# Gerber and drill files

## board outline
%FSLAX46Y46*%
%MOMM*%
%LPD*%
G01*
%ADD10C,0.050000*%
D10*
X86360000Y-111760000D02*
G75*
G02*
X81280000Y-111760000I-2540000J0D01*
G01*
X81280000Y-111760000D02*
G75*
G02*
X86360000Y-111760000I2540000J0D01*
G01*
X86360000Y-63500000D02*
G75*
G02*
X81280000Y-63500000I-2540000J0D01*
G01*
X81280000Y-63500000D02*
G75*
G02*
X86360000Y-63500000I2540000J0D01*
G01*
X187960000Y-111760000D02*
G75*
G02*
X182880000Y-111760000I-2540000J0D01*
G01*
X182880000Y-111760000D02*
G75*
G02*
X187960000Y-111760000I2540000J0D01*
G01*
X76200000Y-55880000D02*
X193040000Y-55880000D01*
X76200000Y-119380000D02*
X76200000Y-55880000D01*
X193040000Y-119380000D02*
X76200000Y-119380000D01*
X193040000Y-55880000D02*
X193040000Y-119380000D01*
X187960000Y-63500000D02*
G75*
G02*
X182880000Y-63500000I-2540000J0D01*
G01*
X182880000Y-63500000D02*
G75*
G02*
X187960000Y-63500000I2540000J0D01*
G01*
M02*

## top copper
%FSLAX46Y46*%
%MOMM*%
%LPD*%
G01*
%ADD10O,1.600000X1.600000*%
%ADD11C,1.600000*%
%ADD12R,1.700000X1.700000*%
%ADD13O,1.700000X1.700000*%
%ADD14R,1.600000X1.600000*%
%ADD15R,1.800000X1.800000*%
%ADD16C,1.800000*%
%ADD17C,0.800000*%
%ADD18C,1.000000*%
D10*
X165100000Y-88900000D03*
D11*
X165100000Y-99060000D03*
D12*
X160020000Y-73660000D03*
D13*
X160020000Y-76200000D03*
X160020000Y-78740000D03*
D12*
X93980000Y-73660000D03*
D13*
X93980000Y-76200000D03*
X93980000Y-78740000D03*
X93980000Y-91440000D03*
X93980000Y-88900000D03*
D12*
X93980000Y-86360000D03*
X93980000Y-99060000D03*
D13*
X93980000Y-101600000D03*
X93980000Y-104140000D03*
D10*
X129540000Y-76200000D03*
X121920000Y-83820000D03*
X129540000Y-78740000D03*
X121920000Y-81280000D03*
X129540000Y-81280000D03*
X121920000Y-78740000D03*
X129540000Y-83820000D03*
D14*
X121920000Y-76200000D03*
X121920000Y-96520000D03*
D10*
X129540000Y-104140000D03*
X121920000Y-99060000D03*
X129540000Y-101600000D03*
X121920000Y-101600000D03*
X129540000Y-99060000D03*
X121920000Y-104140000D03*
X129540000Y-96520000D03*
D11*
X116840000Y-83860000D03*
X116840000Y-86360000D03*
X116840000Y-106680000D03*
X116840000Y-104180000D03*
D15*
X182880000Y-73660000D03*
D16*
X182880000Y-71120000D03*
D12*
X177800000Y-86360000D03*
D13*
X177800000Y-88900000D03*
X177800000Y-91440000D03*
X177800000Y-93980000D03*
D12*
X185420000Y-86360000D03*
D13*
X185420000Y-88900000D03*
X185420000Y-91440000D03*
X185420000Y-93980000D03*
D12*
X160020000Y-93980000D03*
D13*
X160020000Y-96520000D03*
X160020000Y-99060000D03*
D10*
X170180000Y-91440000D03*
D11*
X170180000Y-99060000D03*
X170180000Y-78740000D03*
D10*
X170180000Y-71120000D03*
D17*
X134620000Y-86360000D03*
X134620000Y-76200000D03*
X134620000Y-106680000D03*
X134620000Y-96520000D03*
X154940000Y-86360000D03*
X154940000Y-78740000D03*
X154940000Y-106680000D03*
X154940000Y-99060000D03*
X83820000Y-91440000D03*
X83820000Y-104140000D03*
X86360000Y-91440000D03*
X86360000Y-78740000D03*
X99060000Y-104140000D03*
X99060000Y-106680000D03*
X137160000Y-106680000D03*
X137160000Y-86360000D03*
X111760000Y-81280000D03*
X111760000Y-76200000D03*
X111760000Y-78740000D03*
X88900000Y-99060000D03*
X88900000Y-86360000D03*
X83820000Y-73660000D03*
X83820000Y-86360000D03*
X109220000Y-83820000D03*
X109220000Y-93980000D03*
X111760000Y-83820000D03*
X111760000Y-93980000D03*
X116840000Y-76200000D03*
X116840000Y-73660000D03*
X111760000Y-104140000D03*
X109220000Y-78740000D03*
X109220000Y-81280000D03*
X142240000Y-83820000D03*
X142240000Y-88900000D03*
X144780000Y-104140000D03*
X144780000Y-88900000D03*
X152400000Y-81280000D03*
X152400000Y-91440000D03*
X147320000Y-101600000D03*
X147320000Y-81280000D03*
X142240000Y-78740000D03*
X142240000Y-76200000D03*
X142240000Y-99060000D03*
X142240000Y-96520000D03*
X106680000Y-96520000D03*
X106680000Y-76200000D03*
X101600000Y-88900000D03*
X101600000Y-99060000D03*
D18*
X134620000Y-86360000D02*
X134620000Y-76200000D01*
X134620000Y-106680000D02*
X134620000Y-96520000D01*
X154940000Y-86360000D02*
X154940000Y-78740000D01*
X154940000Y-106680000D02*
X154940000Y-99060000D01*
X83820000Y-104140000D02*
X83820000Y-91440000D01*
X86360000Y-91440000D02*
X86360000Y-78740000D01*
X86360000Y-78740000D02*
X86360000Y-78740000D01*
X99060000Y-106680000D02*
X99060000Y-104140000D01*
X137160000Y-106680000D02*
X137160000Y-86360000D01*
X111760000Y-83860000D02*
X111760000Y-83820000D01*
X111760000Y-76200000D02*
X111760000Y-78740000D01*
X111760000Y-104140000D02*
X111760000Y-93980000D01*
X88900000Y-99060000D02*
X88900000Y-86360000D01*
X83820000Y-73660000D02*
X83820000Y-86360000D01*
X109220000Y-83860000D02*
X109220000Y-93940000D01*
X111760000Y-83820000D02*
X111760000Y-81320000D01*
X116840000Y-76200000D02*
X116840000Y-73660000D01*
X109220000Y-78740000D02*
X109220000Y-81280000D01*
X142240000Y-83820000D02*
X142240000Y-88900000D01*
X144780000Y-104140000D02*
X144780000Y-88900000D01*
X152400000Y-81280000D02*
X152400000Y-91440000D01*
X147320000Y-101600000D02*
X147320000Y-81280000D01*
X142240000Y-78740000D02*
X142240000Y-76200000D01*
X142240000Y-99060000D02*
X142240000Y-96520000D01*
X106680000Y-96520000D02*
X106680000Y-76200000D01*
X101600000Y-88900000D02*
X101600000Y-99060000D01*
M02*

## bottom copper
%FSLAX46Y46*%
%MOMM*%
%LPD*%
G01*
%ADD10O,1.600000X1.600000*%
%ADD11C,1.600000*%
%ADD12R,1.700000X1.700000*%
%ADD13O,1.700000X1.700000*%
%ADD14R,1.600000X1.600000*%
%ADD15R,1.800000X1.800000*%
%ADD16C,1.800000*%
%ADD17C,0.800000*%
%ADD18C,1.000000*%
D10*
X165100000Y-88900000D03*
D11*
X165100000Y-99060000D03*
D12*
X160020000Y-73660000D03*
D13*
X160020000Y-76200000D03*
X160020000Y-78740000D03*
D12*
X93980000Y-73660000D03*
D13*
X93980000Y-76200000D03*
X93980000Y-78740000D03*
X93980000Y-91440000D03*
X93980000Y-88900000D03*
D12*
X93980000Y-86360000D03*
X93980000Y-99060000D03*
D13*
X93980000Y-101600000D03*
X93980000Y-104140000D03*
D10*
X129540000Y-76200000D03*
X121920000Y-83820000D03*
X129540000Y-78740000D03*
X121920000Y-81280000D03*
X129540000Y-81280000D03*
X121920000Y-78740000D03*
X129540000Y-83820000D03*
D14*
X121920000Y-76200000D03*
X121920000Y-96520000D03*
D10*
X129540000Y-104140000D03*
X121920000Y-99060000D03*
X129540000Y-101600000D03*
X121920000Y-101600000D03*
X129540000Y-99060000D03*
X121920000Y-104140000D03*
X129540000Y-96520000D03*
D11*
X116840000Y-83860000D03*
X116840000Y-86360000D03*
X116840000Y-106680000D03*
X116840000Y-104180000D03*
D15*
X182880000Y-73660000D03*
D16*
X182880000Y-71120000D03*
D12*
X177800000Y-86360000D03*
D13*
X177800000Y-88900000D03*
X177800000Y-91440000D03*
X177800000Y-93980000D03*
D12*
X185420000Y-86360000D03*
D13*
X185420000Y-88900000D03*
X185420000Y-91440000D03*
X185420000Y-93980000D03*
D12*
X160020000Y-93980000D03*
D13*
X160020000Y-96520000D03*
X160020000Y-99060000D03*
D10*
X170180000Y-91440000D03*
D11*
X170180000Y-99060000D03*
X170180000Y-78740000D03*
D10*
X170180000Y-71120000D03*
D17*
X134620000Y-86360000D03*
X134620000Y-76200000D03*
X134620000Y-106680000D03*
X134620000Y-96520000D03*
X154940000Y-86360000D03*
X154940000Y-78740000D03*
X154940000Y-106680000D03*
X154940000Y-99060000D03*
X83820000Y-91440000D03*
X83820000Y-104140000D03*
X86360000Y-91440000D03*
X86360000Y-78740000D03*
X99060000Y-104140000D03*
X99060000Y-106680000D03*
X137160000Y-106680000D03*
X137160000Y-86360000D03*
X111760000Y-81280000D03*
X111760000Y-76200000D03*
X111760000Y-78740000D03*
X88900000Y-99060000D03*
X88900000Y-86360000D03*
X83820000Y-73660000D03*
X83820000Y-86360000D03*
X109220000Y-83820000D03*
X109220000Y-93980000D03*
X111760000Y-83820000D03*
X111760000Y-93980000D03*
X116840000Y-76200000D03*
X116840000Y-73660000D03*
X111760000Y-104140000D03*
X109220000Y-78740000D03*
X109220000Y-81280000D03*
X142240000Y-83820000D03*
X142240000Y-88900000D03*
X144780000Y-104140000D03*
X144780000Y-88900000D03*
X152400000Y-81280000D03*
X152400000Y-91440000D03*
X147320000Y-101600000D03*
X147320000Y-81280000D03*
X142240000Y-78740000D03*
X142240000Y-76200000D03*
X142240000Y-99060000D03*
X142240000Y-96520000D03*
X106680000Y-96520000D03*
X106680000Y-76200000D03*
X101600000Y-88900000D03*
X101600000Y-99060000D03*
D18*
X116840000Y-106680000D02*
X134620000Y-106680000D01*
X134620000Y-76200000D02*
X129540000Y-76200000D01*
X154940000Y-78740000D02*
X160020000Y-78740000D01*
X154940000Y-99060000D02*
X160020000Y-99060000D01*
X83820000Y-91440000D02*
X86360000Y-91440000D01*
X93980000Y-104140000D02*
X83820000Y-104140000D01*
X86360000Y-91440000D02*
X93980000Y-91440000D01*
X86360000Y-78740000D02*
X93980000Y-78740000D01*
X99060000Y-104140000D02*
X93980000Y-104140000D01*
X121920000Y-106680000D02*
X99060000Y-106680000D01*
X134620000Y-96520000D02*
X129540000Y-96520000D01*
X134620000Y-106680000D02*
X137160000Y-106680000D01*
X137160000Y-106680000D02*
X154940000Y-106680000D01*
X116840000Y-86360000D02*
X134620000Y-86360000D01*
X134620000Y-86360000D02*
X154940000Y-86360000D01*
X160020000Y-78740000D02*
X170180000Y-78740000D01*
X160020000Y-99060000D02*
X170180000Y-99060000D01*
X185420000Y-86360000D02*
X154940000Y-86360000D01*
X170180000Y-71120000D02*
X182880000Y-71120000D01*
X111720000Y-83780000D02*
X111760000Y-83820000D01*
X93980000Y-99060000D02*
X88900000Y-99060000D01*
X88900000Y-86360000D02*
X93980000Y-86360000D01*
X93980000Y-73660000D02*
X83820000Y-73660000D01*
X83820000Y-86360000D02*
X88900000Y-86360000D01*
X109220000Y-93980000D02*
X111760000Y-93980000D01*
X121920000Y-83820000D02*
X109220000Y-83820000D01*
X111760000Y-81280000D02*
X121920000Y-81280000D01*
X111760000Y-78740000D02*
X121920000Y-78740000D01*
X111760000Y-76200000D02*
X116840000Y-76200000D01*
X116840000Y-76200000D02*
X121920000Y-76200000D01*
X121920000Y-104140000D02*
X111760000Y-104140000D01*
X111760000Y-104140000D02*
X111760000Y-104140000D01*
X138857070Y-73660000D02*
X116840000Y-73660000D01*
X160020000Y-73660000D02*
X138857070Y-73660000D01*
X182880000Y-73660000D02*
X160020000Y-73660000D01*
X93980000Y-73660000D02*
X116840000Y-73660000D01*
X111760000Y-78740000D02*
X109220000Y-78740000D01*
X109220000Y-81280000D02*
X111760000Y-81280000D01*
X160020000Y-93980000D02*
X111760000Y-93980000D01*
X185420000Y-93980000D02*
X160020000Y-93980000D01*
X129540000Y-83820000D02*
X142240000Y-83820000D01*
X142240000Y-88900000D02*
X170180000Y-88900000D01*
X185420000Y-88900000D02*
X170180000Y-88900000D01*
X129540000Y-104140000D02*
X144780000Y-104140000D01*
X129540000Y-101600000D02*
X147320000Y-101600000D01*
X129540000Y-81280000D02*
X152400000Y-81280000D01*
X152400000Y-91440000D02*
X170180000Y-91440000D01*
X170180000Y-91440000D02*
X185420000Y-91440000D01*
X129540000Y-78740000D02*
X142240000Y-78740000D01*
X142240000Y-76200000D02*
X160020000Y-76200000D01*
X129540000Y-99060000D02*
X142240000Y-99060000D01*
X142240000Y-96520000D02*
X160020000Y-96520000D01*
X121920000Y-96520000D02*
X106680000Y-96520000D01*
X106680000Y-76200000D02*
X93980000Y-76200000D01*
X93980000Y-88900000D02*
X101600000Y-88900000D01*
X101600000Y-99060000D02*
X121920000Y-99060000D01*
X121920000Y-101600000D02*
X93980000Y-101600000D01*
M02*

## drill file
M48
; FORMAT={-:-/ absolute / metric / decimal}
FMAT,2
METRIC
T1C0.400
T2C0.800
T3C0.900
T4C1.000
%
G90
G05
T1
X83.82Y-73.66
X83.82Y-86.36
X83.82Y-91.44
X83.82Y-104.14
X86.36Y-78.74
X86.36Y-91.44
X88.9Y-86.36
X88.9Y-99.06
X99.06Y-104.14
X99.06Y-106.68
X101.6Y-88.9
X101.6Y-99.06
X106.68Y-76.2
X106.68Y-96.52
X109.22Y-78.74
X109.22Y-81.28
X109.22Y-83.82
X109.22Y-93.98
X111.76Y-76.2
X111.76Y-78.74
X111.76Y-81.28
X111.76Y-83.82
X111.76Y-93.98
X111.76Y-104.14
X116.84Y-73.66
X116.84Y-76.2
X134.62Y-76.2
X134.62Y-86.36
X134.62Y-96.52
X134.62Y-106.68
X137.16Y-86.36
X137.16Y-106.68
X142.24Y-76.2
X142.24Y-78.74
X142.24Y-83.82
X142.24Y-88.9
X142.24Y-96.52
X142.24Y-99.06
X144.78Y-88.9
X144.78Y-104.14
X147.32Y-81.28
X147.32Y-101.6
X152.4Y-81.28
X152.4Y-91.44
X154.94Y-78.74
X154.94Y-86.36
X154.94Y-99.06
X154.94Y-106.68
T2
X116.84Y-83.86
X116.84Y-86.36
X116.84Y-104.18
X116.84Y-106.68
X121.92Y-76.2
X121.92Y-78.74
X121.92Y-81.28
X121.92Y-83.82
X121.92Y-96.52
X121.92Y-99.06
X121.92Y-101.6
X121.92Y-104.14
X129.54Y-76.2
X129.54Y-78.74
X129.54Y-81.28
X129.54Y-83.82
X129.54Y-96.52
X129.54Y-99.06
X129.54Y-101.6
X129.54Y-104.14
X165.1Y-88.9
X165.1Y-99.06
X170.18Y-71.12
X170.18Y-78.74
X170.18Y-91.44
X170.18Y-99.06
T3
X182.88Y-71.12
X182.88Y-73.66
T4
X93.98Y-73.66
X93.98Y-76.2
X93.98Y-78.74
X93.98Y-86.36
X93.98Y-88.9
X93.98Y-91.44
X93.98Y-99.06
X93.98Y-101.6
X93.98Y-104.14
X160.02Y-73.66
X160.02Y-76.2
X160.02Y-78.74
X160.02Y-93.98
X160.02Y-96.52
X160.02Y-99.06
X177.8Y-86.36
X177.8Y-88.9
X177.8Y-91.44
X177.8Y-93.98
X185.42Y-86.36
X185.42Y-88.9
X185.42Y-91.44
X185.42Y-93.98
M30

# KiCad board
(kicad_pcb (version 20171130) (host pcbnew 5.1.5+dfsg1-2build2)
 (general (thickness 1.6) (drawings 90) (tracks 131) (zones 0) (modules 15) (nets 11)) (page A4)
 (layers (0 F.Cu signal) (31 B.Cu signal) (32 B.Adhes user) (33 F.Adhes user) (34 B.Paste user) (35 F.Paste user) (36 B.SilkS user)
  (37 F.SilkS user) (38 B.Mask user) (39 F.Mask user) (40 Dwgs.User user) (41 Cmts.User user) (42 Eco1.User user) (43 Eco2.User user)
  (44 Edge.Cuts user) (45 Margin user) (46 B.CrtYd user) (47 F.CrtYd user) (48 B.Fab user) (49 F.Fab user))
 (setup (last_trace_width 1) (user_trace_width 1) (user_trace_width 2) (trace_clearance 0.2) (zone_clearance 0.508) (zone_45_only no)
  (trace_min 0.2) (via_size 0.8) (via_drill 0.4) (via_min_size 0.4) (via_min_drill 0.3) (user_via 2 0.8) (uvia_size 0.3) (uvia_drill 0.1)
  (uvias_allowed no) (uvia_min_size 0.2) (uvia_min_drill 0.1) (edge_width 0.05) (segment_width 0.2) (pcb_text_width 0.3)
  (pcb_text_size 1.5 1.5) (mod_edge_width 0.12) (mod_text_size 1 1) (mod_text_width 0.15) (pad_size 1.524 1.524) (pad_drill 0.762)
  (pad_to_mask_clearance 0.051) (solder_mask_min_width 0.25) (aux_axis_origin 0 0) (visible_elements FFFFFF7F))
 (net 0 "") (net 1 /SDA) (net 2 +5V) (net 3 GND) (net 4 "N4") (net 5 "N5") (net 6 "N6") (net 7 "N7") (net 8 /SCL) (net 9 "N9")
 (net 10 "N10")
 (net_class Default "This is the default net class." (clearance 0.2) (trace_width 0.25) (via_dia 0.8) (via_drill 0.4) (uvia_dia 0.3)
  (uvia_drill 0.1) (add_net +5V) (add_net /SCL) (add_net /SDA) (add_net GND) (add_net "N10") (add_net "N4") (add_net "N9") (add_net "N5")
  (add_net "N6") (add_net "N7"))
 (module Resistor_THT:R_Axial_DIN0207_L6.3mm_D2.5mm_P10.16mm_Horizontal (layer F.Cu) (at 165.1 99.06 90)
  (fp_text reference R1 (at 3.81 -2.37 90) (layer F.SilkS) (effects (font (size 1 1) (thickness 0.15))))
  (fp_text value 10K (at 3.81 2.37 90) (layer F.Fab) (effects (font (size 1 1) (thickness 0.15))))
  (pad 2 thru_hole oval (at 10.16 0 90) (size 1.6 1.6) (drill 0.8) (layers *.Cu *.Mask) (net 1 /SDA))
  (pad 1 thru_hole circle (at 0 0 90) (size 1.6 1.6) (drill 0.8) (layers *.Cu *.Mask) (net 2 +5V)))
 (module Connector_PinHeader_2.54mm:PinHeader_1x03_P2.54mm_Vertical (layer F.Cu) (at 160.02 73.66)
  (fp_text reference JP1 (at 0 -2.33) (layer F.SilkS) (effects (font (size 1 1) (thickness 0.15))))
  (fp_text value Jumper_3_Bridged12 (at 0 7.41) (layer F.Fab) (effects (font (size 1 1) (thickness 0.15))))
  (pad 1 thru_hole rect (at 0 0) (size 1.7 1.7) (drill 1) (layers *.Cu *.Mask) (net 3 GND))
  (pad 2 thru_hole oval (at 0 2.54) (size 1.7 1.7) (drill 1) (layers *.Cu *.Mask) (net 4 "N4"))
  (pad 3 thru_hole oval (at 0 5.08) (size 1.7 1.7) (drill 1) (layers *.Cu *.Mask) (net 2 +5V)))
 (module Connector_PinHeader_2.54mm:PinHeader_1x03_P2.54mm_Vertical (layer F.Cu) (at 93.98 73.66)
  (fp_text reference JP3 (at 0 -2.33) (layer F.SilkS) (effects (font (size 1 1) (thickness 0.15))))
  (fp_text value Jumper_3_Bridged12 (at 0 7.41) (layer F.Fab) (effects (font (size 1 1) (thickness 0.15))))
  (pad 1 thru_hole rect (at 0 0) (size 1.7 1.7) (drill 1) (layers *.Cu *.Mask) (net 3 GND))
  (pad 2 thru_hole oval (at 0 2.54) (size 1.7 1.7) (drill 1) (layers *.Cu *.Mask) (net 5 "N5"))
  (pad 3 thru_hole oval (at 0 5.08) (size 1.7 1.7) (drill 1) (layers *.Cu *.Mask) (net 2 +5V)))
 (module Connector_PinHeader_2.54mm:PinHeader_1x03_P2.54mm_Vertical (layer F.Cu) (at 93.98 86.36)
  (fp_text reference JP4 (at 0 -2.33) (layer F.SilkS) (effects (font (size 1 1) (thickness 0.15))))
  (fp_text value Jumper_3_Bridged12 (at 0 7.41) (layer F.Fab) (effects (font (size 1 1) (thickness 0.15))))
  (pad 3 thru_hole oval (at 0 5.08) (size 1.7 1.7) (drill 1) (layers *.Cu *.Mask) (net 2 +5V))
  (pad 2 thru_hole oval (at 0 2.54) (size 1.7 1.7) (drill 1) (layers *.Cu *.Mask) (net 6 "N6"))
  (pad 1 thru_hole rect (at 0 0) (size 1.7 1.7) (drill 1) (layers *.Cu *.Mask) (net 3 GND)))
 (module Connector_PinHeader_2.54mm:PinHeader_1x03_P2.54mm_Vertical (layer F.Cu) (at 93.98 99.06)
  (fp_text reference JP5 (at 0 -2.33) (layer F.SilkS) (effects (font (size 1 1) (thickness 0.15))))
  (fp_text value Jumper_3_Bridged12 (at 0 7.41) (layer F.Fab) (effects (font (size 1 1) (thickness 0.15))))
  (pad 1 thru_hole rect (at 0 0) (size 1.7 1.7) (drill 1) (layers *.Cu *.Mask) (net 3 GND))
  (pad 2 thru_hole oval (at 0 2.54) (size 1.7 1.7) (drill 1) (layers *.Cu *.Mask) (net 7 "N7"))
  (pad 3 thru_hole oval (at 0 5.08) (size 1.7 1.7) (drill 1) (layers *.Cu *.Mask) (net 2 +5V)))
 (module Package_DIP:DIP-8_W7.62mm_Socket (layer F.Cu) (at 121.92 76.2)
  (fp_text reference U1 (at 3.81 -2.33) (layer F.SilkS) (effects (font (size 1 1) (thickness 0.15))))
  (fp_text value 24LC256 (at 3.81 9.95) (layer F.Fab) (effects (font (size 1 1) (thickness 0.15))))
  (pad 8 thru_hole oval (at 7.62 0) (size 1.6 1.6) (drill 0.8) (layers *.Cu *.Mask) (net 2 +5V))
  (pad 4 thru_hole oval (at 0 7.62) (size 1.6 1.6) (drill 0.8) (layers *.Cu *.Mask) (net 3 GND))
  (pad 7 thru_hole oval (at 7.62 2.54) (size 1.6 1.6) (drill 0.8) (layers *.Cu *.Mask) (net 4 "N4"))
  (pad 3 thru_hole oval (at 0 5.08) (size 1.6 1.6) (drill 0.8) (layers *.Cu *.Mask) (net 3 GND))
  (pad 6 thru_hole oval (at 7.62 5.08) (size 1.6 1.6) (drill 0.8) (layers *.Cu *.Mask) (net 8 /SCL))
  (pad 2 thru_hole oval (at 0 2.54) (size 1.6 1.6) (drill 0.8) (layers *.Cu *.Mask) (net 3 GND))
  (pad 5 thru_hole oval (at 7.62 7.62) (size 1.6 1.6) (drill 0.8) (layers *.Cu *.Mask) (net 1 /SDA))
  (pad 1 thru_hole rect (at 0 0) (size 1.6 1.6) (drill 0.8) (layers *.Cu *.Mask) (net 3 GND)))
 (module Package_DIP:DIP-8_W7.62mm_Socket (layer F.Cu) (at 121.92 96.52)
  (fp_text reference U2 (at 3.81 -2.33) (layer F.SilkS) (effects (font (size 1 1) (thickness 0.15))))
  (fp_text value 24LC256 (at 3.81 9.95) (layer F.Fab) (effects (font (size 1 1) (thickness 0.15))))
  (pad 1 thru_hole rect (at 0 0) (size 1.6 1.6) (drill 0.8) (layers *.Cu *.Mask) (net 5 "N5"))
  (pad 5 thru_hole oval (at 7.62 7.62) (size 1.6 1.6) (drill 0.8) (layers *.Cu *.Mask) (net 1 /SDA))
  (pad 2 thru_hole oval (at 0 2.54) (size 1.6 1.6) (drill 0.8) (layers *.Cu *.Mask) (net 6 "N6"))
  (pad 6 thru_hole oval (at 7.62 5.08) (size 1.6 1.6) (drill 0.8) (layers *.Cu *.Mask) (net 8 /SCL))
  (pad 3 thru_hole oval (at 0 5.08) (size 1.6 1.6) (drill 0.8) (layers *.Cu *.Mask) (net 7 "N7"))
  (pad 7 thru_hole oval (at 7.62 2.54) (size 1.6 1.6) (drill 0.8) (layers *.Cu *.Mask) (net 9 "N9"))
  (pad 4 thru_hole oval (at 0 7.62) (size 1.6 1.6) (drill 0.8) (layers *.Cu *.Mask) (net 3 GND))
  (pad 8 thru_hole oval (at 7.62 0) (size 1.6 1.6) (drill 0.8) (layers *.Cu *.Mask) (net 2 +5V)))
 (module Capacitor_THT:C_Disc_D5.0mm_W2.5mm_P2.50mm (layer F.Cu) (at 116.84 86.36 90)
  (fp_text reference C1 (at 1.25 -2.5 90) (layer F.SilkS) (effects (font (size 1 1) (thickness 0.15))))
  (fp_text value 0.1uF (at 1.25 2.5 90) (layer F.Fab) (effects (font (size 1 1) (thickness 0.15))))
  (pad 2 thru_hole circle (at 2.5 0 90) (size 1.6 1.6) (drill 0.8) (layers *.Cu *.Mask) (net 3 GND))
  (pad 1 thru_hole circle (at 0 0 90) (size 1.6 1.6) (drill 0.8) (layers *.Cu *.Mask) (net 2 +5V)))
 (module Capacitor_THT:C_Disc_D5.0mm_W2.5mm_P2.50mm (layer F.Cu) (at 116.84 106.68 90)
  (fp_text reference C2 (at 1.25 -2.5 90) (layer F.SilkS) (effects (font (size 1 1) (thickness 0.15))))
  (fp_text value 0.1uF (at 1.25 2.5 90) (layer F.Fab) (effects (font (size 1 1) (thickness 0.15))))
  (pad 1 thru_hole circle (at 0 0 90) (size 1.6 1.6) (drill 0.8) (layers *.Cu *.Mask) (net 2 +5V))
  (pad 2 thru_hole circle (at 2.5 0 90) (size 1.6 1.6) (drill 0.8) (layers *.Cu *.Mask) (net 3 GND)))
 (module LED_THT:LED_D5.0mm (layer F.Cu) (at 182.88 73.66 90)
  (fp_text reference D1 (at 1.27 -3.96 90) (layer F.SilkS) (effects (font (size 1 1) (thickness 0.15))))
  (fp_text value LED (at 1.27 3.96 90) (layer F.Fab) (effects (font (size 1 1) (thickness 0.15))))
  (pad 1 thru_hole rect (at 0 0 90) (size 1.8 1.8) (drill 0.9) (layers *.Cu *.Mask) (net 3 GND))
  (pad 2 thru_hole circle (at 2.54 0 90) (size 1.8 1.8) (drill 0.9) (layers *.Cu *.Mask) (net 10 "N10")))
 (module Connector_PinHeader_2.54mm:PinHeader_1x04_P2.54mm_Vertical (layer F.Cu) (at 177.8 86.36)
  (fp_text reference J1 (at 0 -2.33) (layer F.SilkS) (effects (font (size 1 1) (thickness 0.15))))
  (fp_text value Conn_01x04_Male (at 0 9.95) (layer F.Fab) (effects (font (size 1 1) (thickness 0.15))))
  (pad 1 thru_hole rect (at 0 0) (size 1.7 1.7) (drill 1) (layers *.Cu *.Mask) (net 2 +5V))
  (pad 2 thru_hole oval (at 0 2.54) (size 1.7 1.7) (drill 1) (layers *.Cu *.Mask) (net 1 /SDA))
  (pad 3 thru_hole oval (at 0 5.08) (size 1.7 1.7) (drill 1) (layers *.Cu *.Mask) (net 8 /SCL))
  (pad 4 thru_hole oval (at 0 7.62) (size 1.7 1.7) (drill 1) (layers *.Cu *.Mask) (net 3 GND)))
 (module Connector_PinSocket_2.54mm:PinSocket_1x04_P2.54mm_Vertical (layer F.Cu) (at 185.42 86.36)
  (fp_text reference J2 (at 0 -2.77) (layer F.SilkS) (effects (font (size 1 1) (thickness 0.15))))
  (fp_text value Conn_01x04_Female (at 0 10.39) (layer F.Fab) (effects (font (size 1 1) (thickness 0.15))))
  (pad 1 thru_hole rect (at 0 0) (size 1.7 1.7) (drill 1) (layers *.Cu *.Mask) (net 2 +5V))
  (pad 2 thru_hole oval (at 0 2.54) (size 1.7 1.7) (drill 1) (layers *.Cu *.Mask) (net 1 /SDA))
  (pad 3 thru_hole oval (at 0 5.08) (size 1.7 1.7) (drill 1) (layers *.Cu *.Mask) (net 8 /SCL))
  (pad 4 thru_hole oval (at 0 7.62) (size 1.7 1.7) (drill 1) (layers *.Cu *.Mask) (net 3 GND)))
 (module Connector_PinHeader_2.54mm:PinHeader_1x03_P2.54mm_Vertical (layer F.Cu) (at 160.02 93.98)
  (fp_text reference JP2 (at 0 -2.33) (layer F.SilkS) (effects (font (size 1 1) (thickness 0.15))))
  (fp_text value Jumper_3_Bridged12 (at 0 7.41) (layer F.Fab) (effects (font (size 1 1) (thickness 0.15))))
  (pad 1 thru_hole rect (at 0 0) (size 1.7 1.7) (drill 1) (layers *.Cu *.Mask) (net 3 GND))
  (pad 2 thru_hole oval (at 0 2.54) (size 1.7 1.7) (drill 1) (layers *.Cu *.Mask) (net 9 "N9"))
  (pad 3 thru_hole oval (at 0 5.08) (size 1.7 1.7) (drill 1) (layers *.Cu *.Mask) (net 2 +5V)))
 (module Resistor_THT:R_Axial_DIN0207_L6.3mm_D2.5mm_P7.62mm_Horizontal (layer F.Cu) (at 170.18 99.06 90)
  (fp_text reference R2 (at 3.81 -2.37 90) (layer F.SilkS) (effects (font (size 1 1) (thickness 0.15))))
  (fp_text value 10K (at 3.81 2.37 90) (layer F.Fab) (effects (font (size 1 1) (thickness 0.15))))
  (pad 2 thru_hole oval (at 7.62 0 90) (size 1.6 1.6) (drill 0.8) (layers *.Cu *.Mask) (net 8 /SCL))
  (pad 1 thru_hole circle (at 0 0 90) (size 1.6 1.6) (drill 0.8) (layers *.Cu *.Mask) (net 2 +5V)))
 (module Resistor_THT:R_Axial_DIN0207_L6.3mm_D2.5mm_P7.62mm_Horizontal (layer F.Cu) (at 170.18 78.74 90)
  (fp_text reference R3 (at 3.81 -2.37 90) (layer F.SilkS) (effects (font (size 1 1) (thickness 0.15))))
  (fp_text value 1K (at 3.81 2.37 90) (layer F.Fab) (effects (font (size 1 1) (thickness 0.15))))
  (pad 1 thru_hole circle (at 0 0 90) (size 1.6 1.6) (drill 0.8) (layers *.Cu *.Mask) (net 2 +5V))
  (pad 2 thru_hole oval (at 7.62 0 90) (size 1.6 1.6) (drill 0.8) (layers *.Cu *.Mask) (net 10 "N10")))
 (gr_circle (center 83.82 111.76) (end 81.28 111.76) (layer Edge.Cuts) (width 0.05))
 (gr_circle (center 83.82 63.5) (end 81.28 63.5) (layer Edge.Cuts) (width 0.05))
 (gr_circle (center 185.42 111.76) (end 182.88 111.76) (layer Edge.Cuts) (width 0.05))
 (gr_line (start 76.2 55.88) (end 193.04 55.88) (layer Edge.Cuts) (width 0.05))
 (gr_line (start 76.2 119.38) (end 76.2 55.88) (layer Edge.Cuts) (width 0.05))
 (gr_line (start 193.04 119.38) (end 76.2 119.38) (layer Edge.Cuts) (width 0.05))
 (gr_line (start 193.04 55.88) (end 193.04 119.38) (layer Edge.Cuts) (width 0.05))
 (gr_circle (center 185.42 63.5) (end 182.88 63.5) (layer Edge.Cuts) (width 0.05))
 (segment (start 116.84 106.68) (end 134.62 106.68) (width 1) (layer B.Cu) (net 2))
 (via (at 134.62 86.36) (size 0.8) (drill 0.4) (layers F.Cu B.Cu) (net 2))
 (segment (start 134.62 86.36) (end 134.62 76.2) (width 1) (layer F.Cu) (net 2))
 (via (at 134.62 76.2) (size 0.8) (drill 0.4) (layers F.Cu B.Cu) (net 2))
 (segment (start 134.62 76.2) (end 129.54 76.2) (width 1) (layer B.Cu) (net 2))
 (via (at 134.62 106.68) (size 0.8) (drill 0.4) (layers F.Cu B.Cu) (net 2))
 (segment (start 134.62 106.68) (end 134.62 96.52) (width 1) (layer F.Cu) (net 2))
 (via (at 134.62 96.52) (size 0.8) (drill 0.4) (layers F.Cu B.Cu) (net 2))
 (via (at 154.94 86.36) (size 0.8) (drill 0.4) (layers F.Cu B.Cu) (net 2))
 (segment (start 154.94 86.36) (end 154.94 78.74) (width 1) (layer F.Cu) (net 2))
 (via (at 154.94 78.74) (size 0.8) (drill 0.4) (layers F.Cu B.Cu) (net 2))
 (segment (start 154.94 78.74) (end 160.02 78.74) (width 1) (layer B.Cu) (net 2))
 (via (at 154.94 106.68) (size 0.8) (drill 0.4) (layers F.Cu B.Cu) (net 2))
 (segment (start 154.94 106.68) (end 154.94 99.06) (width 1) (layer F.Cu) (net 2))
 (via (at 154.94 99.06) (size 0.8) (drill 0.4) (layers F.Cu B.Cu) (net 2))
 (segment (start 154.94 99.06) (end 160.02 99.06) (width 1) (layer B.Cu) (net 2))
 (segment (start 83.82 91.44) (end 86.36 91.44) (width 1) (layer B.Cu) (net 2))
 (via (at 83.82 91.44) (size 0.8) (drill 0.4) (layers F.Cu B.Cu) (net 2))
 (segment (start 83.82 104.14) (end 83.82 91.44) (width 1) (layer F.Cu) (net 2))
 (segment (start 93.98 104.14) (end 83.82 104.14) (width 1) (layer B.Cu) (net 2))
 (via (at 83.82 104.14) (size 0.8) (drill 0.4) (layers F.Cu B.Cu) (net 2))
 (segment (start 86.36 91.44) (end 93.98 91.44) (width 1) (layer B.Cu) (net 2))
 (via (at 86.36 91.44) (size 0.8) (drill 0.4) (layers F.Cu B.Cu) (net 2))
 (segment (start 86.36 91.44) (end 86.36 78.74) (width 1) (layer F.Cu) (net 2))
 (segment (start 86.36 78.74) (end 86.36 78.74) (width 1) (layer F.Cu) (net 2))
 (via (at 86.36 78.74) (size 0.8) (drill 0.4) (layers F.Cu B.Cu) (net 2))
 (segment (start 86.36 78.74) (end 93.98 78.74) (width 1) (layer B.Cu) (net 2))
 (segment (start 99.06 104.14) (end 93.98 104.14) (width 1) (layer B.Cu) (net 2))
 (via (at 99.06 104.14) (size 0.8) (drill 0.4) (layers F.Cu B.Cu) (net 2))
 (segment (start 121.92 106.68) (end 99.06 106.68) (width 1) (layer B.Cu) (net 2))
 (segment (start 99.06 106.68) (end 99.06 104.14) (width 1) (layer F.Cu) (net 2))
 (via (at 99.06 106.68) (size 0.8) (drill 0.4) (layers F.Cu B.Cu) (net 2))
 (segment (start 134.62 96.52) (end 129.54 96.52) (width 1) (layer B.Cu) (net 2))
 (via (at 137.16 106.68) (size 0.8) (drill 0.4) (layers F.Cu B.Cu) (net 2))
 (segment (start 134.62 106.68) (end 137.16 106.68) (width 1) (layer B.Cu) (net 2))
 (segment (start 137.16 106.68) (end 154.94 106.68) (width 1) (layer B.Cu) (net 2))
 (segment (start 137.16 106.68) (end 137.16 86.36) (width 1) (layer F.Cu) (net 2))
 (via (at 137.16 86.36) (size 0.8) (drill 0.4) (layers F.Cu B.Cu) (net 2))
 (segment (start 116.84 86.36) (end 134.62 86.36) (width 1) (layer B.Cu) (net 2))
 (segment (start 134.62 86.36) (end 154.94 86.36) (width 1) (layer B.Cu) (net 2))
 (segment (start 160.02 78.74) (end 170.18 78.74) (width 1) (layer B.Cu) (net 2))
 (segment (start 160.02 99.06) (end 170.18 99.06) (width 1) (layer B.Cu) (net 2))
 (segment (start 185.42 86.36) (end 154.94 86.36) (width 1) (layer B.Cu) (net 2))
 (segment (start 170.18 71.12) (end 182.88 71.12) (width 1) (layer B.Cu) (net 10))
 (segment (start 111.72 83.78) (end 111.76 83.82) (width 1) (layer B.Cu) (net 3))
 (segment (start 111.76 83.86) (end 111.76 83.82) (width 1) (layer F.Cu) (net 3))
 (via (at 111.76 81.28) (size 0.8) (drill 0.4) (layers F.Cu B.Cu) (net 3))
 (via (at 111.76 76.2) (size 0.8) (drill 0.4) (layers F.Cu B.Cu) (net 3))
 (segment (start 111.76 76.2) (end 111.76 78.74) (width 1) (layer F.Cu) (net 3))
 (via (at 111.76 78.74) (size 0.8) (drill 0.4) (layers F.Cu B.Cu) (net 3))
 (segment (start 111.76 104.14) (end 111.76 93.98) (width 1) (layer F.Cu) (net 3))
 (segment (start 93.98 99.06) (end 88.9 99.06) (width 1) (layer B.Cu) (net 3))
 (via (at 88.9 99.06) (size 0.8) (drill 0.4) (layers F.Cu B.Cu) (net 3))
 (segment (start 88.9 99.06) (end 88.9 86.36) (width 1) (layer F.Cu) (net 3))
 (via (at 88.9 86.36) (size 0.8) (drill 0.4) (layers F.Cu B.Cu) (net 3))
 (segment (start 88.9 86.36) (end 93.98 86.36) (width 1) (layer B.Cu) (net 3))
 (segment (start 93.98 73.66) (end 83.82 73.66) (width 1) (layer B.Cu) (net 3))
 (via (at 83.82 73.66) (size 0.8) (drill 0.4) (layers F.Cu B.Cu) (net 3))
 (segment (start 83.82 73.66) (end 83.82 86.36) (width 1) (layer F.Cu) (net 3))
 (via (at 83.82 86.36) (size 0.8) (drill 0.4) (layers F.Cu B.Cu) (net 3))
 (segment (start 83.82 86.36) (end 88.9 86.36) (width 1) (layer B.Cu) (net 3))
 (via (at 109.22 83.82) (size 0.8) (drill 0.4) (layers F.Cu B.Cu) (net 3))
 (segment (start 109.22 83.86) (end 109.22 93.94) (width 1) (layer F.Cu) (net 3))
 (via (at 109.22 93.98) (size 0.8) (drill 0.4) (layers F.Cu B.Cu) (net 3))
 (segment (start 109.22 93.98) (end 111.76 93.98) (width 1) (layer B.Cu) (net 3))
 (segment (start 111.76 83.82) (end 111.76 81.32) (width 1) (layer F.Cu) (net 3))
 (via (at 111.76 83.82) (size 0.8) (drill 0.4) (layers F.Cu B.Cu) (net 3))
 (via (at 111.76 93.98) (size 0.8) (drill 0.4) (layers F.Cu B.Cu) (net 3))
 (segment (start 121.92 83.82) (end 109.22 83.82) (width 1) (layer B.Cu) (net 3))
 (segment (start 111.76 81.28) (end 121.92 81.28) (width 1) (layer B.Cu) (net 3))
 (segment (start 111.76 78.74) (end 121.92 78.74) (width 1) (layer B.Cu) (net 3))
 (segment (start 111.76 76.2) (end 116.84 76.2) (width 1) (layer B.Cu) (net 3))
 (via (at 116.84 76.2) (size 0.8) (drill 0.4) (layers F.Cu B.Cu) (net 3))
 (segment (start 116.84 76.2) (end 121.92 76.2) (width 1) (layer B.Cu) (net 3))
 (segment (start 116.84 76.2) (end 116.84 73.66) (width 1) (layer F.Cu) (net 3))
 (via (at 116.84 73.66) (size 0.8) (drill 0.4) (layers F.Cu B.Cu) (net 3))
 (segment (start 121.92 104.14) (end 111.76 104.14) (width 1) (layer B.Cu) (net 3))
 (segment (start 111.76 104.14) (end 111.76 104.14) (width 1) (layer B.Cu) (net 3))
 (via (at 111.76 104.14) (size 0.8) (drill 0.4) (layers F.Cu B.Cu) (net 3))
 (segment (start 138.85707 73.66) (end 116.84 73.66) (width 1) (layer B.Cu) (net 3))
 (segment (start 160.02 73.66) (end 138.85707 73.66) (width 1) (layer B.Cu) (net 3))
 (segment (start 182.88 73.66) (end 160.02 73.66) (width 1) (layer B.Cu) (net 3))
 (segment (start 93.98 73.66) (end 116.84 73.66) (width 1) (layer B.Cu) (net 3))
 (segment (start 111.76 78.74) (end 109.22 78.74) (width 1) (layer B.Cu) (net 3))
 (via (at 109.22 78.74) (size 0.8) (drill 0.4) (layers F.Cu B.Cu) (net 3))
 (segment (start 109.22 78.74) (end 109.22 81.28) (width 1) (layer F.Cu) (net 3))
 (via (at 109.22 81.28) (size 0.8) (drill 0.4) (layers F.Cu B.Cu) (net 3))
 (segment (start 109.22 81.28) (end 111.76 81.28) (width 1) (layer B.Cu) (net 3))
 (segment (start 160.02 93.98) (end 111.76 93.98) (width 1) (layer B.Cu) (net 3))
 (segment (start 185.42 93.98) (end 160.02 93.98) (width 1) (layer B.Cu) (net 3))
 (via (at 142.24 83.82) (size 0.8) (drill 0.4) (layers F.Cu B.Cu) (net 1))
 (segment (start 142.24 83.82) (end 142.24 88.9) (width 1) (layer F.Cu) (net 1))
 (via (at 142.24 88.9) (size 0.8) (drill 0.4) (layers F.Cu B.Cu) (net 1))
 (segment (start 129.54 83.82) (end 142.24 83.82) (width 1) (layer B.Cu) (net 1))
 (segment (start 142.24 88.9) (end 170.18 88.9) (width 1) (layer B.Cu) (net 1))
 (segment (start 185.42 88.9) (end 170.18 88.9) (width 1) (layer B.Cu) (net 1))
 (segment (start 129.54 104.14) (end 144.78 104.14) (width 1) (layer B.Cu) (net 1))
 (via (at 144.78 104.14) (size 0.8) (drill 0.4) (layers F.Cu B.Cu) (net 1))
 (segment (start 144.78 104.14) (end 144.78 88.9) (width 1) (layer F.Cu) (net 1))
 (via (at 144.78 88.9) (size 0.8) (drill 0.4) (layers F.Cu B.Cu) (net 1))
 (via (at 152.4 81.28) (size 0.8) (drill 0.4) (layers F.Cu B.Cu) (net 8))
 (segment (start 152.4 81.28) (end 152.4 91.44) (width 1) (layer F.Cu) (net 8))
 (via (at 152.4 91.44) (size 0.8) (drill 0.4) (layers F.Cu B.Cu) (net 8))
 (segment (start 129.54 101.6) (end 147.32 101.6) (width 1) (layer B.Cu) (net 8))
 (via (at 147.32 101.6) (size 0.8) (drill 0.4) (layers F.Cu B.Cu) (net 8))
 (segment (start 147.32 101.6) (end 147.32 81.28) (width 1) (layer F.Cu) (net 8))
 (via (at 147.32 81.28) (size 0.8) (drill 0.4) (layers F.Cu B.Cu) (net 8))
 (segment (start 129.54 81.28) (end 152.4 81.28) (width 1) (layer B.Cu) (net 8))
 (segment (start 152.4 91.44) (end 170.18 91.44) (width 1) (layer B.Cu) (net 8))
 (segment (start 170.18 91.44) (end 185.42 91.44) (width 1) (layer B.Cu) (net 8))
 (via (at 142.24 78.74) (size 0.8) (drill 0.4) (layers F.Cu B.Cu) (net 4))
 (segment (start 142.24 78.74) (end 142.24 76.2) (width 1) (layer F.Cu) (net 4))
 (via (at 142.24 76.2) (size 0.8) (drill 0.4) (layers F.Cu B.Cu) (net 4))
 (segment (start 129.54 78.74) (end 142.24 78.74) (width 1) (layer B.Cu) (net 4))
 (segment (start 142.24 76.2) (end 160.02 76.2) (width 1) (layer B.Cu) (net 4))
 (via (at 142.24 99.06) (size 0.8) (drill 0.4) (layers F.Cu B.Cu) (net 9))
 (segment (start 142.24 99.06) (end 142.24 96.52) (width 1) (layer F.Cu) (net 9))
 (via (at 142.24 96.52) (size 0.8) (drill 0.4) (layers F.Cu B.Cu) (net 9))
 (segment (start 129.54 99.06) (end 142.24 99.06) (width 1) (layer B.Cu) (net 9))
 (segment (start 142.24 96.52) (end 160.02 96.52) (width 1) (layer B.Cu) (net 9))
 (segment (start 121.92 96.52) (end 106.68 96.52) (width 1) (layer B.Cu) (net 5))
 (via (at 106.68 96.52) (size 0.8) (drill 0.4) (layers F.Cu B.Cu) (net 5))
 (segment (start 106.68 96.52) (end 106.68 76.2) (width 1) (layer F.Cu) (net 5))
 (via (at 106.68 76.2) (size 0.8) (drill 0.4) (layers F.Cu B.Cu) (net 5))
 (segment (start 106.68 76.2) (end 93.98 76.2) (width 1) (layer B.Cu) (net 5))
 (segment (start 93.98 88.9) (end 101.6 88.9) (width 1) (layer B.Cu) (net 6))
 (via (at 101.6 88.9) (size 0.8) (drill 0.4) (layers F.Cu B.Cu) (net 6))
 (segment (start 101.6 88.9) (end 101.6 99.06) (width 1) (layer F.Cu) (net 6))
 (via (at 101.6 99.06) (size 0.8) (drill 0.4) (layers F.Cu B.Cu) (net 6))
 (segment (start 101.6 99.06) (end 121.92 99.06) (width 1) (layer B.Cu) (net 6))
 (segment (start 121.92 101.6) (end 93.98 101.6) (width 1) (layer B.Cu) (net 7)))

